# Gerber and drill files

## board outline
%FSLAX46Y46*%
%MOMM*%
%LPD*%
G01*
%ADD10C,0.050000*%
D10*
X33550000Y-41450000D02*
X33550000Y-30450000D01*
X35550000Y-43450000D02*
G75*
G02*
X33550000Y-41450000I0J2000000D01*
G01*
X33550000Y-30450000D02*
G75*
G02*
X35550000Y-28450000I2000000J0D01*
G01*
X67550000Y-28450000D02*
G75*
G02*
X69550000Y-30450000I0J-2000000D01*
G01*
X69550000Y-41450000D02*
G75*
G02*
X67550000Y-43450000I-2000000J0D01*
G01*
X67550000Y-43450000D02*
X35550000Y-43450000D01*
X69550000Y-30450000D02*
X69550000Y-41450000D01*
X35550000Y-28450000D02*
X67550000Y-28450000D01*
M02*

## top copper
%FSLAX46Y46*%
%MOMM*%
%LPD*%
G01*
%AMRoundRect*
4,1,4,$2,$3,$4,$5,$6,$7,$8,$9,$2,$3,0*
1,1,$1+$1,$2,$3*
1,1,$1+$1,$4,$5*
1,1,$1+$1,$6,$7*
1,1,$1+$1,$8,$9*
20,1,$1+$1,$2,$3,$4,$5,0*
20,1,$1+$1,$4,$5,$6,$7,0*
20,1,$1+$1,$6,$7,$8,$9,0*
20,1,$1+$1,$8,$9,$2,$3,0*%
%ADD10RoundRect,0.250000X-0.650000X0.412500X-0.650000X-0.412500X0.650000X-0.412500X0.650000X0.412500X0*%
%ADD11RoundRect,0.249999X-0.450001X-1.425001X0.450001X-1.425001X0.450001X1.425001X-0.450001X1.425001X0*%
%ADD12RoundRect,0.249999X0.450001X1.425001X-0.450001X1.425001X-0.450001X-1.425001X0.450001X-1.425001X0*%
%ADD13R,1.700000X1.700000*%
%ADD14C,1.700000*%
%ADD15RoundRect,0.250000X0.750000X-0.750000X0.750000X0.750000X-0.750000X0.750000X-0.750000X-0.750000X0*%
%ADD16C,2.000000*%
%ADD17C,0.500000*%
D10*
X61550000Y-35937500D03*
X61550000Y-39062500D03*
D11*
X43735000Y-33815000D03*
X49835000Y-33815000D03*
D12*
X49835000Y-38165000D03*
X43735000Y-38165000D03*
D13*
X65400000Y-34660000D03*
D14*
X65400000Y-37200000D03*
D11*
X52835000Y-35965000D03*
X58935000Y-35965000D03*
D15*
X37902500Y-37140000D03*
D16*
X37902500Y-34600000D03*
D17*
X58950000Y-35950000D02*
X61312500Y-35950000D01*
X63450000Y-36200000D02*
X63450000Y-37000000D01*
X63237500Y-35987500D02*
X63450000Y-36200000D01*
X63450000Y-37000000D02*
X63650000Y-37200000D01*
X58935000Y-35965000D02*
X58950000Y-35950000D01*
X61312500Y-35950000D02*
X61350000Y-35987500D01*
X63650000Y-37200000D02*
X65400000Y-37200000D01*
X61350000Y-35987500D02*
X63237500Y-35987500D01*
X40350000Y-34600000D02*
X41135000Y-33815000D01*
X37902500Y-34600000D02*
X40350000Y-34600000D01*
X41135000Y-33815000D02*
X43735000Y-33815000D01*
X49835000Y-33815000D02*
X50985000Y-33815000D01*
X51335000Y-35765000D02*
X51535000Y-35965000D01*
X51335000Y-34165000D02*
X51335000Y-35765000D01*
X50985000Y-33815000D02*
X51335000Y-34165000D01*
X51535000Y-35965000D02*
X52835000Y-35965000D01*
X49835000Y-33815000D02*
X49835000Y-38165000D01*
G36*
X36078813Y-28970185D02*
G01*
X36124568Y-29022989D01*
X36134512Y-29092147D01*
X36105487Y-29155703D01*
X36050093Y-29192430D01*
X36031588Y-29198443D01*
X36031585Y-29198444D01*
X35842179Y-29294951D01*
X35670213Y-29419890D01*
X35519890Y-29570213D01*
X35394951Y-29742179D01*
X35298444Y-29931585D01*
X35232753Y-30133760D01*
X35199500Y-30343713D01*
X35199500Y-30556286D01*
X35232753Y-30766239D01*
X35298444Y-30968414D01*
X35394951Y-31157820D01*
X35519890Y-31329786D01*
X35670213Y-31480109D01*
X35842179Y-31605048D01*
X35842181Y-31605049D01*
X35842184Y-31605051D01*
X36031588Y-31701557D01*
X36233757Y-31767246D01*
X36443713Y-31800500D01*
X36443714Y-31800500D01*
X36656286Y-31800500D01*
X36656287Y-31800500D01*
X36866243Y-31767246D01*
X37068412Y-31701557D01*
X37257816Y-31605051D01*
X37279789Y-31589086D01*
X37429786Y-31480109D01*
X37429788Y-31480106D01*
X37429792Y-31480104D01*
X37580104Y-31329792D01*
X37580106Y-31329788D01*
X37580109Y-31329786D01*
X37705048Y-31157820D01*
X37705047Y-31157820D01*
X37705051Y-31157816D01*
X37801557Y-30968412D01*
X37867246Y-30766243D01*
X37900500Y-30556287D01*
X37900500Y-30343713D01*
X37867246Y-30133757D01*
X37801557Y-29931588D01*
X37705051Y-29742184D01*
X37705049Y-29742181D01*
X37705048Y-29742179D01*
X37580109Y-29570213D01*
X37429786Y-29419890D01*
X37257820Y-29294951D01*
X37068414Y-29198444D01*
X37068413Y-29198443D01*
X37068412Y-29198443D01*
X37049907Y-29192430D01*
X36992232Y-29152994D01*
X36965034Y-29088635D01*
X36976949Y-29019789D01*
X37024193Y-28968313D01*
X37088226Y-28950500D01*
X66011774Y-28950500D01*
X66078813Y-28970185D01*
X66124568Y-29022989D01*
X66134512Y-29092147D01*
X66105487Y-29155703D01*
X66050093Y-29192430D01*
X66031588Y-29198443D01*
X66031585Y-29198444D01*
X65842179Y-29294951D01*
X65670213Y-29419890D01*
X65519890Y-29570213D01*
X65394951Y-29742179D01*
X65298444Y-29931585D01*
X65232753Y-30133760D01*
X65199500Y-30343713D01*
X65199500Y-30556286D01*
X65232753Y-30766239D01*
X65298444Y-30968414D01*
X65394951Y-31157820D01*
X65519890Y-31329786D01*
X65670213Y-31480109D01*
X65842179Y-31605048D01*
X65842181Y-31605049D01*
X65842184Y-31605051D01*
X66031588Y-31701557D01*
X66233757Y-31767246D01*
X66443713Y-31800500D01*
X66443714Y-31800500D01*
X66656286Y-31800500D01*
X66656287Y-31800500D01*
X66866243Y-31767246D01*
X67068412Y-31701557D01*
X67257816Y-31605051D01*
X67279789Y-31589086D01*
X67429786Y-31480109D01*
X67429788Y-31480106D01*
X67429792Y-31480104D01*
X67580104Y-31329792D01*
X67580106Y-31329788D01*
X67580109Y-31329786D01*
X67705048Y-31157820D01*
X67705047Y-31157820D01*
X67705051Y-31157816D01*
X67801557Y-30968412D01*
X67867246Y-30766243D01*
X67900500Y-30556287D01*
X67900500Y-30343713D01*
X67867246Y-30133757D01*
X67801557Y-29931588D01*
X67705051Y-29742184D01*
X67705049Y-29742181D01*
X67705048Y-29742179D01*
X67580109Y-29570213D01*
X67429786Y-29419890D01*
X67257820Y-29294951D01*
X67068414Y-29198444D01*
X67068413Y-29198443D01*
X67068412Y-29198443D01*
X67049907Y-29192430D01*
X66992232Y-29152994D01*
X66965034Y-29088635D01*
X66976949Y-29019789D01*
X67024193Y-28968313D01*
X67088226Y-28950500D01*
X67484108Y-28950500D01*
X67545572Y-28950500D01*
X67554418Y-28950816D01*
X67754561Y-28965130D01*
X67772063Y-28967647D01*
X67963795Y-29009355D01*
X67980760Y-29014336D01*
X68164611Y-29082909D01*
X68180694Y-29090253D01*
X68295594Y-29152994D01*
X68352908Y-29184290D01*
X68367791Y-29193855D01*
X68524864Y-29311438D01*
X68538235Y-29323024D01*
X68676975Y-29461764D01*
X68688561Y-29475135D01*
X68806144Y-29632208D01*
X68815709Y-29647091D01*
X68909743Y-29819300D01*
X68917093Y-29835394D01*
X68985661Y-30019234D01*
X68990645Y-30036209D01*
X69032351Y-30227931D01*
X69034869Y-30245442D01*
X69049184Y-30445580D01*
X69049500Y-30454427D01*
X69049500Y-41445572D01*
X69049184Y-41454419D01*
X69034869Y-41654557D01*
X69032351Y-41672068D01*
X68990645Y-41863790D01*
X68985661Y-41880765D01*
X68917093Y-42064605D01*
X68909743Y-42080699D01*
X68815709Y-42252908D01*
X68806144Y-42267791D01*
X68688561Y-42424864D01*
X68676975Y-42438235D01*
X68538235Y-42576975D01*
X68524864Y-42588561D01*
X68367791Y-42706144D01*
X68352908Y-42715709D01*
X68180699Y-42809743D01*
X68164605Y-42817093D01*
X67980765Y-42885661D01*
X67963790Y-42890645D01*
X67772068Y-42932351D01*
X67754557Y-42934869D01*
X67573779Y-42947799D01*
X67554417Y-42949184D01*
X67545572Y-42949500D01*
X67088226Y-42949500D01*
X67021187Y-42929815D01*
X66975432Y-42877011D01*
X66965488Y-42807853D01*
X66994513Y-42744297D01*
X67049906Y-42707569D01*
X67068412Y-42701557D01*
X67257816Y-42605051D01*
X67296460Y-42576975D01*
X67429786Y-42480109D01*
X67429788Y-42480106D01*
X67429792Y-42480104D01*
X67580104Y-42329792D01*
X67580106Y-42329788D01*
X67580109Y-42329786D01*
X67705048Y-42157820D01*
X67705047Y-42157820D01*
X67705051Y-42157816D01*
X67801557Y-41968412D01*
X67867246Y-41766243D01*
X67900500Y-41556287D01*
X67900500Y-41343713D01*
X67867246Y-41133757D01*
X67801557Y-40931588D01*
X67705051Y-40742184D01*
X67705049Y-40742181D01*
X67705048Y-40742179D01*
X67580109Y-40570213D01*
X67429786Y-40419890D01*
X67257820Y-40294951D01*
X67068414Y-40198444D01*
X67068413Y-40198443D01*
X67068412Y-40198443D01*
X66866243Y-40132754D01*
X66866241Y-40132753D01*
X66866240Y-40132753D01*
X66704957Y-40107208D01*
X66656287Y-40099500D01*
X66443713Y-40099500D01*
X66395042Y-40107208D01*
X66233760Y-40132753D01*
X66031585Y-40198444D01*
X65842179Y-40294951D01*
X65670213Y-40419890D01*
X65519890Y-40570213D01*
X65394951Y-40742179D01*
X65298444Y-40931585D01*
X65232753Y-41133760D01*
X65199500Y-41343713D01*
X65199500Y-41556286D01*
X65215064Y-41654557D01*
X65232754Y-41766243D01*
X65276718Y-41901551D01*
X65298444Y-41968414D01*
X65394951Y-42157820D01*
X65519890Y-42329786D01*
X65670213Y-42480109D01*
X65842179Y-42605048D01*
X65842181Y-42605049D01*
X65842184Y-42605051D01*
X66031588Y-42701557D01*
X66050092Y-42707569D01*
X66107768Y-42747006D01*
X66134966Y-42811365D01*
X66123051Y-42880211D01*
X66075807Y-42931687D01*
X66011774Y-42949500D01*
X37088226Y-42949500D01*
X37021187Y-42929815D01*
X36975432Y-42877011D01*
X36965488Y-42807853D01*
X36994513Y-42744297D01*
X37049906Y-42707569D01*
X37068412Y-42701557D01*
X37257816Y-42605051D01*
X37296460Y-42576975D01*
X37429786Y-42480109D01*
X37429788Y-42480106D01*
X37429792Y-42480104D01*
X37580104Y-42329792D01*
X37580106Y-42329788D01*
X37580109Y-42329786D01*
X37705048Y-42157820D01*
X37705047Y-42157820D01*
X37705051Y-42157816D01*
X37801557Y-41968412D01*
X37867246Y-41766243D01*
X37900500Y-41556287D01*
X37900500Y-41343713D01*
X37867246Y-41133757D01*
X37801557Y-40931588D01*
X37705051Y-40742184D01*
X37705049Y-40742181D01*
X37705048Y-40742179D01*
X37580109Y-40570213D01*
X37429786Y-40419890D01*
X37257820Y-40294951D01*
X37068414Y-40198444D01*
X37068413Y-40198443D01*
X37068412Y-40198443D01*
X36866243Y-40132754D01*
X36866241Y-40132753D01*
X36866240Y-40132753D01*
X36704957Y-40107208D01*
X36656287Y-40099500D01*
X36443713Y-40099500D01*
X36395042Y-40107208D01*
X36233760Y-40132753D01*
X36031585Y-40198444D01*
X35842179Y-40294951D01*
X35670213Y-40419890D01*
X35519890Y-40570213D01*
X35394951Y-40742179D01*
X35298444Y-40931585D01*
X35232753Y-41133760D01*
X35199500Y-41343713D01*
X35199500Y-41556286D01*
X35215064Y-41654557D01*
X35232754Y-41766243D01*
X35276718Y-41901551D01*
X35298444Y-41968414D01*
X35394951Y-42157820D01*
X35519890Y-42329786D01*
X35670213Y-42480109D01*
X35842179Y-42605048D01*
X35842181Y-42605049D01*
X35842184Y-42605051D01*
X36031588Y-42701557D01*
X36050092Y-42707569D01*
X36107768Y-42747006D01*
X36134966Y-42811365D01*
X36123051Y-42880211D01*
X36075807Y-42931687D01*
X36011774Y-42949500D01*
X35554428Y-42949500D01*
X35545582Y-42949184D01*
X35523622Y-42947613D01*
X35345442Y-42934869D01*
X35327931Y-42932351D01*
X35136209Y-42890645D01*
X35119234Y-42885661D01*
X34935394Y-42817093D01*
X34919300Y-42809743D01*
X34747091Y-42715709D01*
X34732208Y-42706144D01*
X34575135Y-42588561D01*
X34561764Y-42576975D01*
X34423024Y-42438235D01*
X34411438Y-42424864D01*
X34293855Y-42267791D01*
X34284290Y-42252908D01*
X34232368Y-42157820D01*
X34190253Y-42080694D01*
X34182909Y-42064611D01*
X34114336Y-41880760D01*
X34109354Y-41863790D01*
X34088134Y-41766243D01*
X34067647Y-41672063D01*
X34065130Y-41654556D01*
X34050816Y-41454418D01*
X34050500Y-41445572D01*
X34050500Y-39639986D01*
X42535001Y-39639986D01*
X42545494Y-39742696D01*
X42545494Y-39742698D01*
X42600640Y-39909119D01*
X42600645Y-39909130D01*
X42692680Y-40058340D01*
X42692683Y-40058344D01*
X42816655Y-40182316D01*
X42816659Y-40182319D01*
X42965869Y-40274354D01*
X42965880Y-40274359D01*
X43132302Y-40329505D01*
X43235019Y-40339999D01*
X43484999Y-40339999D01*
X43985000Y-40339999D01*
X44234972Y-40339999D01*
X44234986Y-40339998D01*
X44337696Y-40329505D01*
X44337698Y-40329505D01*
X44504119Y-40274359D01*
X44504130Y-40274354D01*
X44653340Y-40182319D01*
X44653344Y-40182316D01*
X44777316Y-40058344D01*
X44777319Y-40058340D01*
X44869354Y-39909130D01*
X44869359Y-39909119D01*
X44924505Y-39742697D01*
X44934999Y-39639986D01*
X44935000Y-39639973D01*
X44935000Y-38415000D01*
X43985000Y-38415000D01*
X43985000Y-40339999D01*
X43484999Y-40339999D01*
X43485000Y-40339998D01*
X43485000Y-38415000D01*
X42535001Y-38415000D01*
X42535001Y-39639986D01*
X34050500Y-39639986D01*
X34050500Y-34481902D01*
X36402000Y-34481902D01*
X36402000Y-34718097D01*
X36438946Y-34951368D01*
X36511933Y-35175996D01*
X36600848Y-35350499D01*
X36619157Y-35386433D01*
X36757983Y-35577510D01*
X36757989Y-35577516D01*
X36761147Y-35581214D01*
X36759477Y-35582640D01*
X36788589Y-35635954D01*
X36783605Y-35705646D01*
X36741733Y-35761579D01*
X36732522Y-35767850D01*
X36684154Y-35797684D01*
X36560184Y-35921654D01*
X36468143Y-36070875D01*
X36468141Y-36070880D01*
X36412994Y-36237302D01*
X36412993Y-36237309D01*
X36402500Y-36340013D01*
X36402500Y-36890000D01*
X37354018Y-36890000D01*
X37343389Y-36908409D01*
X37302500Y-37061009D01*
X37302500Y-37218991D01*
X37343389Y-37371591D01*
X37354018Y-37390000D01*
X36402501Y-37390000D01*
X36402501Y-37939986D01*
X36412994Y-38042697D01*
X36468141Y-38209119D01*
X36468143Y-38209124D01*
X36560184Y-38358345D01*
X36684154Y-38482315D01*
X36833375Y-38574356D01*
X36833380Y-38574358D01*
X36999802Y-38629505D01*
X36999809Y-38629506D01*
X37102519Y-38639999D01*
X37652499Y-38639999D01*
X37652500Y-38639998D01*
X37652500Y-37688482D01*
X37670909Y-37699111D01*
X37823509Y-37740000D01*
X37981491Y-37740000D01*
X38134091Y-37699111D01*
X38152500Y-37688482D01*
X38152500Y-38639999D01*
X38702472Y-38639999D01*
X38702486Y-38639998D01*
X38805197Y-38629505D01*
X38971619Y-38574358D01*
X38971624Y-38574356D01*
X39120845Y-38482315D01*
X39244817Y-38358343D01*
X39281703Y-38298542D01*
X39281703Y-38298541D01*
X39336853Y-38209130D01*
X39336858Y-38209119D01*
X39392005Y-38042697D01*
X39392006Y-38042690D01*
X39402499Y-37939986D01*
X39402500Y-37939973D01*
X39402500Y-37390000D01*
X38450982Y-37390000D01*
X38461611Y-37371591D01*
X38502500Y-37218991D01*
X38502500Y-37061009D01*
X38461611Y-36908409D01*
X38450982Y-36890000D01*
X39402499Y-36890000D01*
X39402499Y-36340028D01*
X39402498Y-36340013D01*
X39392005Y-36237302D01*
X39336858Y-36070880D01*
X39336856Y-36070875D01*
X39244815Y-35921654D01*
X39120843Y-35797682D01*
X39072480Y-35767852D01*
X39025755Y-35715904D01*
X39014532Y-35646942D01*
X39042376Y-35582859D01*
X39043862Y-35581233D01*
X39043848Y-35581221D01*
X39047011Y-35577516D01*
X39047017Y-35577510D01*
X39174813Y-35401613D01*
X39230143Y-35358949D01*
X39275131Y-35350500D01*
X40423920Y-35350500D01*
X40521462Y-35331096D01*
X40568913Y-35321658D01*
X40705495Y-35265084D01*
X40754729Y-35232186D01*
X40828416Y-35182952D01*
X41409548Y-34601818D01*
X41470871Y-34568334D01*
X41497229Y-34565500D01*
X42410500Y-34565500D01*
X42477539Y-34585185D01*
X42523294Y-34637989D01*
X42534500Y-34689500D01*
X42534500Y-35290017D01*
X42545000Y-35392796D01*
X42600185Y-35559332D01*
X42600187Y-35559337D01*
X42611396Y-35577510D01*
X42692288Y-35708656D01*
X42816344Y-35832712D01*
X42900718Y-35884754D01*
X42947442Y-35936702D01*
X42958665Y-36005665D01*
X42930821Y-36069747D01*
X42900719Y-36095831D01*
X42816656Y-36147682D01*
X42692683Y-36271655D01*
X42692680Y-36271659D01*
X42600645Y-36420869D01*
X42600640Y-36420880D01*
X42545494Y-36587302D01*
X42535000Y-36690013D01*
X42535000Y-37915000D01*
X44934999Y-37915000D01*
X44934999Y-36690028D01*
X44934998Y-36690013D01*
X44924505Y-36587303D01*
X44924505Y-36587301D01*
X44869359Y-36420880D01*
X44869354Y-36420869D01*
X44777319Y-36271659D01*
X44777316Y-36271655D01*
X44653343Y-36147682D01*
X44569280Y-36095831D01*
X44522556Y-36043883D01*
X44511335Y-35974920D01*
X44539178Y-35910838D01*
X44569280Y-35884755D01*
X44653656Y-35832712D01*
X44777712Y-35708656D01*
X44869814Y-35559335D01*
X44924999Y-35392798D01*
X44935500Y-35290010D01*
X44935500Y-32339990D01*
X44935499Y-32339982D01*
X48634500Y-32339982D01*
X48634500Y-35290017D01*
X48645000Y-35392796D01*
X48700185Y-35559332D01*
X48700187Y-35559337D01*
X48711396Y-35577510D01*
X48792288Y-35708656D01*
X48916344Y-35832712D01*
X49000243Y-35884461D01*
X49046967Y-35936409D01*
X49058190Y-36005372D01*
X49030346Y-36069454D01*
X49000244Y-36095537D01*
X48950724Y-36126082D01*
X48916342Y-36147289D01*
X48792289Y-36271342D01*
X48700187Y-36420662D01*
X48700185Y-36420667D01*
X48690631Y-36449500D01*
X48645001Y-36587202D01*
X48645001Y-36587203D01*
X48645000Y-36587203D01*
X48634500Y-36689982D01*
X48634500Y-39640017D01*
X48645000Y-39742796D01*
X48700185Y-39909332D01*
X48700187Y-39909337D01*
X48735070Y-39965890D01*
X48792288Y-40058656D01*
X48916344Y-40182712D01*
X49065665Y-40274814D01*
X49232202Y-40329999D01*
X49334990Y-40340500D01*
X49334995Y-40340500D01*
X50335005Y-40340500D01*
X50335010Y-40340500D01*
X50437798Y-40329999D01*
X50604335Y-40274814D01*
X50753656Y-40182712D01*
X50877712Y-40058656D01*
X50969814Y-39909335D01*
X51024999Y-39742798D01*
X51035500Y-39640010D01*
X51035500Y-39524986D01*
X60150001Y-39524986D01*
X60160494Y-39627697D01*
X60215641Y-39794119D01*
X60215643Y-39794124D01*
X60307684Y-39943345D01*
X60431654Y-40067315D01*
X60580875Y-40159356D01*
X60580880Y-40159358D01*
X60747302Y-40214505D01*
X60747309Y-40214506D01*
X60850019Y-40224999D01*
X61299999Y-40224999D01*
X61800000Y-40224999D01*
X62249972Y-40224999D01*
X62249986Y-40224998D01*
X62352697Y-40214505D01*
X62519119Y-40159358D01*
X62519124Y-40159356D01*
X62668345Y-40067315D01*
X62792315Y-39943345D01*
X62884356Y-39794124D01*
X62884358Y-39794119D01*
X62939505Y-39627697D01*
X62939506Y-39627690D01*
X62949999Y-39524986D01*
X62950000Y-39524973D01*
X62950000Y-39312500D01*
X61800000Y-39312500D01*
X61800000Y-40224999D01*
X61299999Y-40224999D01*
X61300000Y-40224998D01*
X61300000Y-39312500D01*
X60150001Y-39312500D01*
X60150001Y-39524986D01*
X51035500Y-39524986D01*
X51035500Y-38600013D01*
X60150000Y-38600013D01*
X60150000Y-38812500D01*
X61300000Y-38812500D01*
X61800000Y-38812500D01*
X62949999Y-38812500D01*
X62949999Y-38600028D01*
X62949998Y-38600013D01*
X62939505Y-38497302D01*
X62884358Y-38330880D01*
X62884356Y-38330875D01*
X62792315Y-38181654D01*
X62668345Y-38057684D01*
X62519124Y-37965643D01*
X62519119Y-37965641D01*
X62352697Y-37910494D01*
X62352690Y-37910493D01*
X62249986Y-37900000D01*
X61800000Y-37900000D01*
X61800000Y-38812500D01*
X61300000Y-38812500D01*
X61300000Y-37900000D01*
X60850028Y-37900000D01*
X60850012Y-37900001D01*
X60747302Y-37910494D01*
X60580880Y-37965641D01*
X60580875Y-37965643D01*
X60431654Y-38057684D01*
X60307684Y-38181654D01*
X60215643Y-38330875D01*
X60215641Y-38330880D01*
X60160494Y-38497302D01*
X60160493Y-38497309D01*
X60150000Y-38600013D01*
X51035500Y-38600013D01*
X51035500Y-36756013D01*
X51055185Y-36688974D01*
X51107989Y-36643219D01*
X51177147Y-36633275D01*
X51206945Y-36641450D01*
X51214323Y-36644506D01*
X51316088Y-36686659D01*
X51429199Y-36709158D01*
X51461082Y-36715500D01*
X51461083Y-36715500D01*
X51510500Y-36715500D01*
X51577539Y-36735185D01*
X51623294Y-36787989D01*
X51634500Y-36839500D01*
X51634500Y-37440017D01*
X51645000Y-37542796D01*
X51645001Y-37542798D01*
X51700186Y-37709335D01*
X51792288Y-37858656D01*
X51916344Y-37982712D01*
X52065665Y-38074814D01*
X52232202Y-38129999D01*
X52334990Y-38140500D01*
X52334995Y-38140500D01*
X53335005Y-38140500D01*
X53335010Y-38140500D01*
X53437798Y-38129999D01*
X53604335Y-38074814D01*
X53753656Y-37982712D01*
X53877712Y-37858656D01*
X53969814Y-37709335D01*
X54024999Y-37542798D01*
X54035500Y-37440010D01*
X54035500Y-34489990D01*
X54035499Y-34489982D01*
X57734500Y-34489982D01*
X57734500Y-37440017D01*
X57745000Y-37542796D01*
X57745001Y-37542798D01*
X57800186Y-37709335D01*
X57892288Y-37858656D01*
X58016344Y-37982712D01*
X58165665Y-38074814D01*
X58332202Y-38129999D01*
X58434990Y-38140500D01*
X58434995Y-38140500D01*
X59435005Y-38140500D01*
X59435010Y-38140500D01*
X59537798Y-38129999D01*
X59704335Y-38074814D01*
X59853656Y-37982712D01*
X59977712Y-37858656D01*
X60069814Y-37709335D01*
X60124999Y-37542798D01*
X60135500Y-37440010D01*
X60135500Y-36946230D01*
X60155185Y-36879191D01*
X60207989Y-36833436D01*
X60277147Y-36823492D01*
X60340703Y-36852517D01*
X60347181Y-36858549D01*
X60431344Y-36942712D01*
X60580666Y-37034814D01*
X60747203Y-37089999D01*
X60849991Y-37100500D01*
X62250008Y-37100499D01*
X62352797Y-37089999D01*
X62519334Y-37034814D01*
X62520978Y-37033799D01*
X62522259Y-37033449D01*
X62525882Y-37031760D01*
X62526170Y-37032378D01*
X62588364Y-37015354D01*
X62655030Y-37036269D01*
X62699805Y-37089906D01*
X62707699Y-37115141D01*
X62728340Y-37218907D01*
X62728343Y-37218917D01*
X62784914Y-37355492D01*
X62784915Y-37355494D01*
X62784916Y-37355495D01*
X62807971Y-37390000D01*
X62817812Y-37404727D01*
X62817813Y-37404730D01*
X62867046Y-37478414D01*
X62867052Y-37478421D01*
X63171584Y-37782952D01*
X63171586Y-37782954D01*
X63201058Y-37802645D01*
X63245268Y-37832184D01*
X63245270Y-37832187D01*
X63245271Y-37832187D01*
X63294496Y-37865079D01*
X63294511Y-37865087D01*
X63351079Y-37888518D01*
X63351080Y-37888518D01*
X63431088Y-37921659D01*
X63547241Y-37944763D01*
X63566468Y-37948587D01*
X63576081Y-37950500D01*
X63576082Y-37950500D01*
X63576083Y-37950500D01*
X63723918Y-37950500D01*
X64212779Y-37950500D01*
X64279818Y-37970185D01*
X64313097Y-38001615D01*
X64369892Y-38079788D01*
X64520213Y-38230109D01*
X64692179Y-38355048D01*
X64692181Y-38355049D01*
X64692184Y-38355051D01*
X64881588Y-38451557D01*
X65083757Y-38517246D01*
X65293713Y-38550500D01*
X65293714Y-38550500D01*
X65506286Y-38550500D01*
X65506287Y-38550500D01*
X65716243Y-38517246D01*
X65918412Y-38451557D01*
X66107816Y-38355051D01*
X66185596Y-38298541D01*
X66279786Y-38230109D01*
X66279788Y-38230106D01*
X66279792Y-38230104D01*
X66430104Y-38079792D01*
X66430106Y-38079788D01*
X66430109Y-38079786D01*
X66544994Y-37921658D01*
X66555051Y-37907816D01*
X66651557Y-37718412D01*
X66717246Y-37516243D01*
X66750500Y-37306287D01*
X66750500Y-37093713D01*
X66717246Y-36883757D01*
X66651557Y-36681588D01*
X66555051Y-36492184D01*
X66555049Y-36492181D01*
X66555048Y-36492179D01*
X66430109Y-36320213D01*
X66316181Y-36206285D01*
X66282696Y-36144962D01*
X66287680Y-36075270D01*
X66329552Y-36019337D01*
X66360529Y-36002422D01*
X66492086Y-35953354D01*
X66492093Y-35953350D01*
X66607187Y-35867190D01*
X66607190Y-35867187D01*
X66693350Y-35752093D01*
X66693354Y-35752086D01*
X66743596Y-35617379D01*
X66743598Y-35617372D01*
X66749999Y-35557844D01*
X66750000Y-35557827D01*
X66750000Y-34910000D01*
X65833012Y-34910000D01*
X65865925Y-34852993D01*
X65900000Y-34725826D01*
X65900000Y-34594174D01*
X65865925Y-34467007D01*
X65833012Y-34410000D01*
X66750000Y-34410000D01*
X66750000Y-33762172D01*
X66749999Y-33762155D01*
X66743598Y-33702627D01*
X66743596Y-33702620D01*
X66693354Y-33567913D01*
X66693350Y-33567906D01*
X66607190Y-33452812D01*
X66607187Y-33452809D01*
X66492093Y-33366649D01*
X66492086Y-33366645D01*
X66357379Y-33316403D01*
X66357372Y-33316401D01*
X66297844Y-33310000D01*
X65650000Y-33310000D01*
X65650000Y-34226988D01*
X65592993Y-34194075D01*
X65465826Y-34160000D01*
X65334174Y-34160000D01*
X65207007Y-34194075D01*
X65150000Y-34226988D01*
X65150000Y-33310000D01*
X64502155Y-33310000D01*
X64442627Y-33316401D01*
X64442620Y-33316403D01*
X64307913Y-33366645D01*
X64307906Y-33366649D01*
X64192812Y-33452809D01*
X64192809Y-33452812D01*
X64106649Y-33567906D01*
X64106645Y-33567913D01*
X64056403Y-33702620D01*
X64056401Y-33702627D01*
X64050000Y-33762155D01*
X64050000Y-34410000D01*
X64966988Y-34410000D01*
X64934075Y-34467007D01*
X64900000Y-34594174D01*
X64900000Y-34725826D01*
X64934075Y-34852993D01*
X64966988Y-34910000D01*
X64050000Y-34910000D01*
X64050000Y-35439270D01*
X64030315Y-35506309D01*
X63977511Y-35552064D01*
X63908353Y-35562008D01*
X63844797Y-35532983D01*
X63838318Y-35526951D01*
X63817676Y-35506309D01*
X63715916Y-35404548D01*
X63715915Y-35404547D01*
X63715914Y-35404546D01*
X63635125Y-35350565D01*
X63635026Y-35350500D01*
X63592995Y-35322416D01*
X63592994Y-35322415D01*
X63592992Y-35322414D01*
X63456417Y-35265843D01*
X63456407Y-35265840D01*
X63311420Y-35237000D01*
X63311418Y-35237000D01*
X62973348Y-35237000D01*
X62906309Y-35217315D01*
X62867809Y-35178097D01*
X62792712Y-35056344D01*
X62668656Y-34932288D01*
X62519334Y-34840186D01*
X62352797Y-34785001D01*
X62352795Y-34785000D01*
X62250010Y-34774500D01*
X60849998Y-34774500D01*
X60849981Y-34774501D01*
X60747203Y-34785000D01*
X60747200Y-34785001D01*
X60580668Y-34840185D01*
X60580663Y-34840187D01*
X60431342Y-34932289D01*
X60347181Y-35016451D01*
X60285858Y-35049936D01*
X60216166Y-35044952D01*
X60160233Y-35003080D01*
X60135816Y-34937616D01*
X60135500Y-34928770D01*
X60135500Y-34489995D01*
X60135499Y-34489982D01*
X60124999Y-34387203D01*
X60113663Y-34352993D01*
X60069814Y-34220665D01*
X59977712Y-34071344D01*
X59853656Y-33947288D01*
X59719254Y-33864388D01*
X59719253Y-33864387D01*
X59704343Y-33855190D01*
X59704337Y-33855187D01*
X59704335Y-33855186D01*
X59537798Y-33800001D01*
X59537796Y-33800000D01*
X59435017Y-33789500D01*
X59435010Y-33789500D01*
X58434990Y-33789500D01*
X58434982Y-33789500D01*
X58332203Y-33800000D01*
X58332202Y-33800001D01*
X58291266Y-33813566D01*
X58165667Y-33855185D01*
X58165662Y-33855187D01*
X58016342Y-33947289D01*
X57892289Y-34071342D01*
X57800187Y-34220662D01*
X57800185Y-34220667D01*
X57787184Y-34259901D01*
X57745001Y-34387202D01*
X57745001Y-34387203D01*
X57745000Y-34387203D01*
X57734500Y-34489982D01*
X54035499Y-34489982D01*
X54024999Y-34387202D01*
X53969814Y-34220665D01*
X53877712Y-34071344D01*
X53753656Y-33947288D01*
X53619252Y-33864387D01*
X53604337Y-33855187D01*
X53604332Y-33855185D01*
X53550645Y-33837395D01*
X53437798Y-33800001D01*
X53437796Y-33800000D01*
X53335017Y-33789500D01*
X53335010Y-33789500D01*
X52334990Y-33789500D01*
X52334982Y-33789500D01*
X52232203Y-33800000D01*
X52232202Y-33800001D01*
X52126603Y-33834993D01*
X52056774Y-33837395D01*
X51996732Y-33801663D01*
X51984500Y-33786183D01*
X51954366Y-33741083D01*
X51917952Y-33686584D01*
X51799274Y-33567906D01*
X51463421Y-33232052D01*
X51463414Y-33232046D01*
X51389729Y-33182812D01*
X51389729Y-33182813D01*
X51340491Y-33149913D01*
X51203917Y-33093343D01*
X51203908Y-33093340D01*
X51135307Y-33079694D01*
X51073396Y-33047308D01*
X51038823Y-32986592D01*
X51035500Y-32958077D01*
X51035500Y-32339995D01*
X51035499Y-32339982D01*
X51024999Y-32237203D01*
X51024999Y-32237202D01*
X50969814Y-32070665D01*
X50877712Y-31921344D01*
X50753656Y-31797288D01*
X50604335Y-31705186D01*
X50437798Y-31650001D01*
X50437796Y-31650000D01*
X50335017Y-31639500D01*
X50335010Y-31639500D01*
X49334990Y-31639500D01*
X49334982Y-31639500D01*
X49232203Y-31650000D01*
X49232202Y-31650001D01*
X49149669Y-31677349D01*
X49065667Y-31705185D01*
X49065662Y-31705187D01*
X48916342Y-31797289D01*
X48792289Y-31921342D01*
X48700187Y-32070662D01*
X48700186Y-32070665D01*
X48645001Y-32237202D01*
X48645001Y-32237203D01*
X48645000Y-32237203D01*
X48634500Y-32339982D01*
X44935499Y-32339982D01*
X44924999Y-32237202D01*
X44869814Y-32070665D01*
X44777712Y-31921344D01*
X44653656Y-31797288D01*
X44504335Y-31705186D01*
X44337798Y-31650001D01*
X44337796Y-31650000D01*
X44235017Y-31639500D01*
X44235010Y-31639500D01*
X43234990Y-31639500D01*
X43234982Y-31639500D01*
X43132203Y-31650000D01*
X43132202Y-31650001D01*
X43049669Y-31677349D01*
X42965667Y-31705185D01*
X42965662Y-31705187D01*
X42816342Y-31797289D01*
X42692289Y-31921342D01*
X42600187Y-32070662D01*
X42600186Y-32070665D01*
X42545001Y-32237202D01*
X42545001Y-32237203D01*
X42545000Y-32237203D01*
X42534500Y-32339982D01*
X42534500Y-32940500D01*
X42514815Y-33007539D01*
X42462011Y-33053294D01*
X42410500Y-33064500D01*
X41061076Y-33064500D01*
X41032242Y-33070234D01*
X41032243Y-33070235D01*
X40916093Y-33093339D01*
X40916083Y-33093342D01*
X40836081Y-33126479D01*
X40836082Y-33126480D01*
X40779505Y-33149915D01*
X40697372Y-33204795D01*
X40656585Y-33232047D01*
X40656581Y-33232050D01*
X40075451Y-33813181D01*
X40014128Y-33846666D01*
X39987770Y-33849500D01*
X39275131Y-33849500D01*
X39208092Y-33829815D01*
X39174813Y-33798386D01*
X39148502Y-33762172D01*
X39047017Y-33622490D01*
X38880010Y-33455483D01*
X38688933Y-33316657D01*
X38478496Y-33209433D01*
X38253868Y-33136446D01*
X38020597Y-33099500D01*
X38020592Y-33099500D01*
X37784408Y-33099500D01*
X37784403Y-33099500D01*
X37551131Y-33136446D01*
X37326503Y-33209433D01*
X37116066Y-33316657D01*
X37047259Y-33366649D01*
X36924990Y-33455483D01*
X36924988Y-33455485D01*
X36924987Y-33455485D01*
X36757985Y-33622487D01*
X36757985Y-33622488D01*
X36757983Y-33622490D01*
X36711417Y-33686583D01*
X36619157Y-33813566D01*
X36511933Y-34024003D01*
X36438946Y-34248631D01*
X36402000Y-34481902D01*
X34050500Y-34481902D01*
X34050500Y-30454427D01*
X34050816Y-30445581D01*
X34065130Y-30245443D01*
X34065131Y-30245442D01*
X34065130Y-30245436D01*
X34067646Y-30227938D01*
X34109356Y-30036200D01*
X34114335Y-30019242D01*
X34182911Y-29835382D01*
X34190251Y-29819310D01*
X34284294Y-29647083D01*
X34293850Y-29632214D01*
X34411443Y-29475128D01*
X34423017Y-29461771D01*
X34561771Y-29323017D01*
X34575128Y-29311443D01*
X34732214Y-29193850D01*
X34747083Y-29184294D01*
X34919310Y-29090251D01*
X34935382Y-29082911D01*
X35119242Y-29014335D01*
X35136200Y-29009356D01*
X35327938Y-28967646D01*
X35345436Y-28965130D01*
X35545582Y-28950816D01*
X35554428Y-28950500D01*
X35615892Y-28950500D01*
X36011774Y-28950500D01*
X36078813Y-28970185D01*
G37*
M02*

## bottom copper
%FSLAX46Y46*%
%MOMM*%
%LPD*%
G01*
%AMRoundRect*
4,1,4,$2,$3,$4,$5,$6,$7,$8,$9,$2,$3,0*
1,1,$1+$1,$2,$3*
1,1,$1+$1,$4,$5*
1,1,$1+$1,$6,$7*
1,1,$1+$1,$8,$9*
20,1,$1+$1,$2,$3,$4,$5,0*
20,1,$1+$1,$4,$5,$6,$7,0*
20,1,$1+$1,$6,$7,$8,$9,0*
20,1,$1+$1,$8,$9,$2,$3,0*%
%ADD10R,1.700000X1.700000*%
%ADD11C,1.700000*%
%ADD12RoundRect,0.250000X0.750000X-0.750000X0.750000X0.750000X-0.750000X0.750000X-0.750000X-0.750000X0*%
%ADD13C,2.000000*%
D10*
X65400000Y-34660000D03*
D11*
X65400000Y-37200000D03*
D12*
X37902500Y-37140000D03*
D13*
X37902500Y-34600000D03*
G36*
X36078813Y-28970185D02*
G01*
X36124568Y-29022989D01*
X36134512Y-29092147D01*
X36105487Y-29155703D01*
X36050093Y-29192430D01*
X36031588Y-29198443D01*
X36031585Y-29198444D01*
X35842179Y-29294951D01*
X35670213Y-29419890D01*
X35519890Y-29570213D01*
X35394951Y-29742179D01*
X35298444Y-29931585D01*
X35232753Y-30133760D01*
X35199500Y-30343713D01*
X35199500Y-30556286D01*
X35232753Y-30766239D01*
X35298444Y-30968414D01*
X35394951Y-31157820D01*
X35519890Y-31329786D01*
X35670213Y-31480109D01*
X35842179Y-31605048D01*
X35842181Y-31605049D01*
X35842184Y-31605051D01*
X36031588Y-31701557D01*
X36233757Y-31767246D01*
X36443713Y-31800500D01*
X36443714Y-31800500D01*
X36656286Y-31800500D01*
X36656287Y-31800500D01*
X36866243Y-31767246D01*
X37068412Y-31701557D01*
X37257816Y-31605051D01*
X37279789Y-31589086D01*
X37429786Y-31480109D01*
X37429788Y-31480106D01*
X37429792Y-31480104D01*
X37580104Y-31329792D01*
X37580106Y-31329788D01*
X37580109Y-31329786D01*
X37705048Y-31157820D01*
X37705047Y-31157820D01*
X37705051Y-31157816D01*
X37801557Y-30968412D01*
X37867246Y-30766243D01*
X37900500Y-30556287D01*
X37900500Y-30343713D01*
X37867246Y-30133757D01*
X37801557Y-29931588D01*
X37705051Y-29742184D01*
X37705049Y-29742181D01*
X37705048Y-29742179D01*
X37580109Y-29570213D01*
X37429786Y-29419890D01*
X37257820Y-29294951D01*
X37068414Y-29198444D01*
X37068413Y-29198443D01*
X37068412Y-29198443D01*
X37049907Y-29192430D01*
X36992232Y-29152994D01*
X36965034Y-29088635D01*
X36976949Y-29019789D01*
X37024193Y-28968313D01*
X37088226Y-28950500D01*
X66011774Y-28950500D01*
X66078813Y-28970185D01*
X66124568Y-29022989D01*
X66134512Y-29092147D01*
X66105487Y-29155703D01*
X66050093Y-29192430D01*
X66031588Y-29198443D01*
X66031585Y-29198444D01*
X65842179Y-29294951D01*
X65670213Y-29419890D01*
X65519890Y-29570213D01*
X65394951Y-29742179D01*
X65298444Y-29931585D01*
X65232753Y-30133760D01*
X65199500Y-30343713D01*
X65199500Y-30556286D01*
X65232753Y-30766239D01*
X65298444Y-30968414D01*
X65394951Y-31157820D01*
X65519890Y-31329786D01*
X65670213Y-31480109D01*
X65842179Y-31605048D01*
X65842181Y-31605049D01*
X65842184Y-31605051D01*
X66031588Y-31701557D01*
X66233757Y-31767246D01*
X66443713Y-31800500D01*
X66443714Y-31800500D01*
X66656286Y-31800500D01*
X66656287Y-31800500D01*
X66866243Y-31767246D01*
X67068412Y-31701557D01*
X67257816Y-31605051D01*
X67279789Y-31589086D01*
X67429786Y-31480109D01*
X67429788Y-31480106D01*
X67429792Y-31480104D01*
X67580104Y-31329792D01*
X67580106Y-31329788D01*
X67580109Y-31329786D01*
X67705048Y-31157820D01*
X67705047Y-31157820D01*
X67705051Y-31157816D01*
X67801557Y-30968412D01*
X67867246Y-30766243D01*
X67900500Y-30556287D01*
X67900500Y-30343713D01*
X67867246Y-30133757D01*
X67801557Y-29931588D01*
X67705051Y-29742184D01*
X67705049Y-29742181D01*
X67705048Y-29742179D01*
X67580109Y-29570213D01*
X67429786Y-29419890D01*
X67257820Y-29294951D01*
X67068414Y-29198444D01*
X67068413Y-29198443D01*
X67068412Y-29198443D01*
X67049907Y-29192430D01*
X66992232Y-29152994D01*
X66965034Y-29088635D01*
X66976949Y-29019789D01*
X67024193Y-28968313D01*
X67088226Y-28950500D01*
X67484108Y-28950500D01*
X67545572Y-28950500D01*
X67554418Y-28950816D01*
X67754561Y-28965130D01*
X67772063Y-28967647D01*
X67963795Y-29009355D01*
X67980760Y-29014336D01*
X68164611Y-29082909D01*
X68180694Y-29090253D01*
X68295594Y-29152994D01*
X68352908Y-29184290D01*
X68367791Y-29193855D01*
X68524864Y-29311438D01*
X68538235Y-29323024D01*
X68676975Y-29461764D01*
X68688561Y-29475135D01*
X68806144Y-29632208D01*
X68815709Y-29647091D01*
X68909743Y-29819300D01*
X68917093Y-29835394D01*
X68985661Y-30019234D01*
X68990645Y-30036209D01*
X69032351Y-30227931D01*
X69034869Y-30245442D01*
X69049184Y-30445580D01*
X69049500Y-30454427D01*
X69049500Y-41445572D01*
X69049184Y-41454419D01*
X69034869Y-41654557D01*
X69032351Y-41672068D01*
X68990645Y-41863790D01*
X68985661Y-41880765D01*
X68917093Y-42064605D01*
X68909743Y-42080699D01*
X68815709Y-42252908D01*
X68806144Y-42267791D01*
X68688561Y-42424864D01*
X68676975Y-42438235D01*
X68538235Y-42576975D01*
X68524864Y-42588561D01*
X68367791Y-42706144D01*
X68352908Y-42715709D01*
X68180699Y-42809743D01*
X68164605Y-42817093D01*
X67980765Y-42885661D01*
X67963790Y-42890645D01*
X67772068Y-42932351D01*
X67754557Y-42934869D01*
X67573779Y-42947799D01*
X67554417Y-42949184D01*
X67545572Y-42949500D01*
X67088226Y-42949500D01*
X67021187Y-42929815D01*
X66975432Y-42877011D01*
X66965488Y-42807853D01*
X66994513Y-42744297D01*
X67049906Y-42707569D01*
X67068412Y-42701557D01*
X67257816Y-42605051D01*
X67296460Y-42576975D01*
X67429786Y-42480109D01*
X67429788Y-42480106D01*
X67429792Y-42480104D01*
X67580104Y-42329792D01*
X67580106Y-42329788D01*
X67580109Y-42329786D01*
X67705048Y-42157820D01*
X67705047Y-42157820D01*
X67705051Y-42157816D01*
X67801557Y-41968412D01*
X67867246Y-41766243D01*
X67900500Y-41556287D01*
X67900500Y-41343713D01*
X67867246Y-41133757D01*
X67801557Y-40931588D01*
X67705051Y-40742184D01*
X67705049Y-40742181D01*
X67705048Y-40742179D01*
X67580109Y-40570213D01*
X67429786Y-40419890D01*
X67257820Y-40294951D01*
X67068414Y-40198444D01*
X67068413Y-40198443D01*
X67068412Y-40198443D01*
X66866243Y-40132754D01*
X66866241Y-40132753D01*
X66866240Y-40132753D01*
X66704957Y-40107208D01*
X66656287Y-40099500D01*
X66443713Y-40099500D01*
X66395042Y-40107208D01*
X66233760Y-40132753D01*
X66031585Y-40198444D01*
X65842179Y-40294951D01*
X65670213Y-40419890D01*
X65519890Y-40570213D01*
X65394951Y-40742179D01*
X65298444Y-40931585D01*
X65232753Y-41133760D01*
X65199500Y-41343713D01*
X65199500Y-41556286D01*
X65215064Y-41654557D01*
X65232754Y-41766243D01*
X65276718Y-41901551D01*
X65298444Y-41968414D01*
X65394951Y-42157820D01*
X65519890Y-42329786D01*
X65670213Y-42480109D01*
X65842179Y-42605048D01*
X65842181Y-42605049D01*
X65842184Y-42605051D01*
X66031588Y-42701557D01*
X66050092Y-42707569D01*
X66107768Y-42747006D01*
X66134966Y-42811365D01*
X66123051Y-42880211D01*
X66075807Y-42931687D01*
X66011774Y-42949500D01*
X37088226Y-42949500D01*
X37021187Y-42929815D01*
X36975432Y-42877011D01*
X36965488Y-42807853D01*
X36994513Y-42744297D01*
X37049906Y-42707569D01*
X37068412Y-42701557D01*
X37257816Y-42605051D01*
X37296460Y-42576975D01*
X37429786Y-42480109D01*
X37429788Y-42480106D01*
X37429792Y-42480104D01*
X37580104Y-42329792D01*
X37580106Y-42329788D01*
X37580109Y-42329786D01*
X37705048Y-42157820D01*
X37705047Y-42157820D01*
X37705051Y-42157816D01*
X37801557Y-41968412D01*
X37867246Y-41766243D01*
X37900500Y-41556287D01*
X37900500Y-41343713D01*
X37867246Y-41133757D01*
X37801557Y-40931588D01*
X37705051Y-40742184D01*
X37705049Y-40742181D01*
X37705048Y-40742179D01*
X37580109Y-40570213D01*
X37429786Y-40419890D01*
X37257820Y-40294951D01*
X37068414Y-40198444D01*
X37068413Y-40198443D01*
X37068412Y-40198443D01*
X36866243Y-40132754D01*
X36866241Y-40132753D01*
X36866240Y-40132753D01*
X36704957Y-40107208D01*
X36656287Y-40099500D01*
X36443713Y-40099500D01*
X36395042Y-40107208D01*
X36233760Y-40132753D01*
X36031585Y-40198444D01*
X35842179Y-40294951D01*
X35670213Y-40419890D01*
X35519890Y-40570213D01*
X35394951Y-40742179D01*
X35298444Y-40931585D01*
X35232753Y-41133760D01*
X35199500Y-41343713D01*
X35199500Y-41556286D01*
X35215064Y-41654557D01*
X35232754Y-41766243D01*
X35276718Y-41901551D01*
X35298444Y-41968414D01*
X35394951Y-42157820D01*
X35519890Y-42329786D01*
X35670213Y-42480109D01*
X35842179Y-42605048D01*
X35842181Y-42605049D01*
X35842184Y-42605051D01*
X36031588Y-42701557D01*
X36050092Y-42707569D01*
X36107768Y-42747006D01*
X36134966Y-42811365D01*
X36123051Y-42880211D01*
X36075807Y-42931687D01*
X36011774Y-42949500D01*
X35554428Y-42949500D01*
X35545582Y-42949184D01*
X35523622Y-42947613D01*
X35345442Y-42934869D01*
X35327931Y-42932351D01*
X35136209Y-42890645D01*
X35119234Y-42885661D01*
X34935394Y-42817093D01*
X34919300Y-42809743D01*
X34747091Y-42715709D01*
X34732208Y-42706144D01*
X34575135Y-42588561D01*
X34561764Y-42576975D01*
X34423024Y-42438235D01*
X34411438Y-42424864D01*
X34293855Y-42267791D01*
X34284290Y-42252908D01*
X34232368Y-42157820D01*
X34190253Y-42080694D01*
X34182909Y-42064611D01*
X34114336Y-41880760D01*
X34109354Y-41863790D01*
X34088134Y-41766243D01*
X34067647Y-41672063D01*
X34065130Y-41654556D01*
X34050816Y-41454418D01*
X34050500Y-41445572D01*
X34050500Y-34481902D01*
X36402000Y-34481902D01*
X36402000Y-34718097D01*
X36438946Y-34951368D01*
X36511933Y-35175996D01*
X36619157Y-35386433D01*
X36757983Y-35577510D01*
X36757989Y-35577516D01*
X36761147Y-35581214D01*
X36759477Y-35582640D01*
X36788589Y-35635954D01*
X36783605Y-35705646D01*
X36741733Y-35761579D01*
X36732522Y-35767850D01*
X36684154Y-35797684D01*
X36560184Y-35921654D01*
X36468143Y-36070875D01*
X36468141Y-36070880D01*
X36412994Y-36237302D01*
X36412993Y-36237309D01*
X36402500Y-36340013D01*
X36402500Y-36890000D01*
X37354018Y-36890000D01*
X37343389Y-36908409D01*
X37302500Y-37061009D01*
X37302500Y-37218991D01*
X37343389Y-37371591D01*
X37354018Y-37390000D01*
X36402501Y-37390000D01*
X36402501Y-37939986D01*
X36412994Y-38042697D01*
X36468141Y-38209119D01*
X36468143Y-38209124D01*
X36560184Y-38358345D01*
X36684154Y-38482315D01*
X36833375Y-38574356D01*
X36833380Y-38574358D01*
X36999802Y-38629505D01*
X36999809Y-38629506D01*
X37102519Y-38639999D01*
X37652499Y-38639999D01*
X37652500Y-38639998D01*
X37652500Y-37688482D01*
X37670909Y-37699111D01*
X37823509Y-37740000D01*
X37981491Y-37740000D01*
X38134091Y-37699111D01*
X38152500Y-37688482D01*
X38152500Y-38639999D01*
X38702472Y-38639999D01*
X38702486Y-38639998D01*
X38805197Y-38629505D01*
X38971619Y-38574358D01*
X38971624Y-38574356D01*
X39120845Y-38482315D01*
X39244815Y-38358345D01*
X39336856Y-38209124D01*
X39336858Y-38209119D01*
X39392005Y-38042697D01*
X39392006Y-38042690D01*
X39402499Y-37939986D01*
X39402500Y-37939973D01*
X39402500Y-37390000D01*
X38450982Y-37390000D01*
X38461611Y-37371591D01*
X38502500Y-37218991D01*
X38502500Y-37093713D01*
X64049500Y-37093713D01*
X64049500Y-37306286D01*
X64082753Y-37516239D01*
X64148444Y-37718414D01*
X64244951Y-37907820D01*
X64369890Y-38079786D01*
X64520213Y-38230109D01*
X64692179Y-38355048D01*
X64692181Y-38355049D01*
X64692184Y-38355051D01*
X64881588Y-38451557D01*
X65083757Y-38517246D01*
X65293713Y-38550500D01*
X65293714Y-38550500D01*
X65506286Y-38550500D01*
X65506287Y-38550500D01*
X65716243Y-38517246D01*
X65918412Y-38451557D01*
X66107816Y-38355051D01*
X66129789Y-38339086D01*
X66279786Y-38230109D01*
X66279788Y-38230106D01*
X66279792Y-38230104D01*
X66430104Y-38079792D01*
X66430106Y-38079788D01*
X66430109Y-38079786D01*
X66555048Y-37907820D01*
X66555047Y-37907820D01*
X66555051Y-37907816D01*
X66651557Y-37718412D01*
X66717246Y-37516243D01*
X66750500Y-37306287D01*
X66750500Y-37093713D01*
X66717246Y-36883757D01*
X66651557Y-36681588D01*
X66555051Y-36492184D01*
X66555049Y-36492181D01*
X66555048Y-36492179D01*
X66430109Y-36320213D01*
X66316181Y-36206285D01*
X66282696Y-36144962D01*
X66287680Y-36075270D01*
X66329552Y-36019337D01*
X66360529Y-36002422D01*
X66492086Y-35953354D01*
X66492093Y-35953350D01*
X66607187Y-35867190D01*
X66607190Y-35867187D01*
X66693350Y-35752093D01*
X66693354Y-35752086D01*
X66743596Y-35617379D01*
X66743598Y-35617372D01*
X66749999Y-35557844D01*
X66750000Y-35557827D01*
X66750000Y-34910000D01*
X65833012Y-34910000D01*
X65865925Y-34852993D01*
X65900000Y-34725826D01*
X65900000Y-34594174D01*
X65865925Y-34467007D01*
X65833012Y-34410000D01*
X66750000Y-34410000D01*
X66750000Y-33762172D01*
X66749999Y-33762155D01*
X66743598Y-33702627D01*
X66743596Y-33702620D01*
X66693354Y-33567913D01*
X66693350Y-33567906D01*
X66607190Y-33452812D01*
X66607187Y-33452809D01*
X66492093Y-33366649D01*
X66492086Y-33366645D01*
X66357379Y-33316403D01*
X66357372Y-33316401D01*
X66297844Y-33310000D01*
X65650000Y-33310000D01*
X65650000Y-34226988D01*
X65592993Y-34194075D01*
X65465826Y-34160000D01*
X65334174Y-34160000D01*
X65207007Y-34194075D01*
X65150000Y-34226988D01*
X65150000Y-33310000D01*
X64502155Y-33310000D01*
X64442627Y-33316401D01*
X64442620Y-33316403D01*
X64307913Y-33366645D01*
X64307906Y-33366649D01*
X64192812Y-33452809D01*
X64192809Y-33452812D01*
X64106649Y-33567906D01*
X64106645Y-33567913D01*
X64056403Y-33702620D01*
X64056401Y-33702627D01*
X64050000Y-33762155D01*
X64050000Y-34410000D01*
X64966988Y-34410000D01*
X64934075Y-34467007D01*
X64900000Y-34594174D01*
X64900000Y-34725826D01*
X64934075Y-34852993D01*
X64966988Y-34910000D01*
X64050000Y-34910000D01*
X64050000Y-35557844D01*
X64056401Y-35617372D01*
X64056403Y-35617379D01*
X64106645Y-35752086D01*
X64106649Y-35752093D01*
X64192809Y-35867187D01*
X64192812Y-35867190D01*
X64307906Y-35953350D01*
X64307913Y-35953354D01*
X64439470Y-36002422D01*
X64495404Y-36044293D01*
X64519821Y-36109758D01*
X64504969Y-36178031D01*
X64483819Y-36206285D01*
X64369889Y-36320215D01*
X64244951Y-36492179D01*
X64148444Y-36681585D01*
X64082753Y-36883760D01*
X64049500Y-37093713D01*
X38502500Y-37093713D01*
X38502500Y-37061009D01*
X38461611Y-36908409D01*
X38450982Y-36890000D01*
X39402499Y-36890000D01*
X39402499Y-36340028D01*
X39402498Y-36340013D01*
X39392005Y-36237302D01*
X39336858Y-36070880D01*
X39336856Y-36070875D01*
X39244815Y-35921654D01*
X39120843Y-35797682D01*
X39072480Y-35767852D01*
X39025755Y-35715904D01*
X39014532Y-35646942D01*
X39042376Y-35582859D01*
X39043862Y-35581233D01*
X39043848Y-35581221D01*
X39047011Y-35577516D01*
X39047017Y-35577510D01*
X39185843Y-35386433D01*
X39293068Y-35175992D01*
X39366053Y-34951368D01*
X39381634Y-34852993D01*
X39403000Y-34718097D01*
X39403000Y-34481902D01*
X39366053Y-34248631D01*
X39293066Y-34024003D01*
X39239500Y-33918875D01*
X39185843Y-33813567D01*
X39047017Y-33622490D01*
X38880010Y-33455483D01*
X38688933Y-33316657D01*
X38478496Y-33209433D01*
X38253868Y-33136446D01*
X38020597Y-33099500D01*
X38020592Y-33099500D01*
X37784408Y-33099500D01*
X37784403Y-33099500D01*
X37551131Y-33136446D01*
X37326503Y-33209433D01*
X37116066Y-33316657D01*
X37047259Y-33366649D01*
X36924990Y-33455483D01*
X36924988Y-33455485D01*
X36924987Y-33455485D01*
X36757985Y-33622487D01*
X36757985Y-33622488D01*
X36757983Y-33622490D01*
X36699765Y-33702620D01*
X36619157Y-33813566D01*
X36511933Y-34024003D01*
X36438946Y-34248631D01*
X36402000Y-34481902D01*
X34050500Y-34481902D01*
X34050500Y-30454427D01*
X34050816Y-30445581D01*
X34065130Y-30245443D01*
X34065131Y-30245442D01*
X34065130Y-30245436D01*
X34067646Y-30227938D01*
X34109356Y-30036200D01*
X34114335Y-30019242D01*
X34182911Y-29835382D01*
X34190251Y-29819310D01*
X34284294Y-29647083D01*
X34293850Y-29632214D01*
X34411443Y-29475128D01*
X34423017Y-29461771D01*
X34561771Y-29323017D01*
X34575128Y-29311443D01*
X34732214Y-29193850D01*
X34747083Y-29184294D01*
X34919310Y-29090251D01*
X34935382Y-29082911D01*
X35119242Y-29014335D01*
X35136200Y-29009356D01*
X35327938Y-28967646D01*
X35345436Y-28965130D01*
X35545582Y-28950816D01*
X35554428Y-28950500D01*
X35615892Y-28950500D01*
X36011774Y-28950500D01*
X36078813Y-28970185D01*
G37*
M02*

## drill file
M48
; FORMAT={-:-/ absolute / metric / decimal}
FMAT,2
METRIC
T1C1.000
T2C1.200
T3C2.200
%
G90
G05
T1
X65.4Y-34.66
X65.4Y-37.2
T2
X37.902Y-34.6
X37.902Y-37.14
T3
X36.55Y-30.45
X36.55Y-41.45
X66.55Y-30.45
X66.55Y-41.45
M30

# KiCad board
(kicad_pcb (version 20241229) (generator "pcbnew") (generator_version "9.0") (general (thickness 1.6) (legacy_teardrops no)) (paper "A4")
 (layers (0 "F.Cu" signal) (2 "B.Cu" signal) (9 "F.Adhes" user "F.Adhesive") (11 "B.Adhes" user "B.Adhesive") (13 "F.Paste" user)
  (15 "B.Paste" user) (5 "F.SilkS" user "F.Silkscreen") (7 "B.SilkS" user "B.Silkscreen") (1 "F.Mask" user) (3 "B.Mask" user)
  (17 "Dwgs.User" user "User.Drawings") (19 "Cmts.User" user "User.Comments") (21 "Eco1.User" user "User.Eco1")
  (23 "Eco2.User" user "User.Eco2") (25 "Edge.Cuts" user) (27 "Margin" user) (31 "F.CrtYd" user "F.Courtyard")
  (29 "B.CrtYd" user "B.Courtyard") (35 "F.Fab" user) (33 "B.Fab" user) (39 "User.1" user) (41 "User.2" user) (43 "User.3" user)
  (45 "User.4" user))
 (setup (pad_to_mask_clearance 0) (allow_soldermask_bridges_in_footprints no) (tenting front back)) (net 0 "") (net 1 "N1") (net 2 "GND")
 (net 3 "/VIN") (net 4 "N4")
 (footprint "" (layer "F.Cu") (at 36.55 30.45)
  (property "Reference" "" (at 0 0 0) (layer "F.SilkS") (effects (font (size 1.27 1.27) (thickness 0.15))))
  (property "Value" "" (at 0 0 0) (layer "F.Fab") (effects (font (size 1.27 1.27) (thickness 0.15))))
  (pad "" np_thru_hole circle (at 0 0) (size 2.2 2.2) (drill 2.2) (layers "*.Cu" "*.Mask")))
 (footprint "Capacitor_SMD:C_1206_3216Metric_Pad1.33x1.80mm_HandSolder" (layer "F.Cu") (at 61.55 37.5 -90)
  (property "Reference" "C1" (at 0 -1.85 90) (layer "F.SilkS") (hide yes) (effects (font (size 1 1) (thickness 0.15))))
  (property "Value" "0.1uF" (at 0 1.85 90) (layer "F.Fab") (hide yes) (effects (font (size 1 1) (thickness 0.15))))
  (pad "1" smd roundrect (at -1.5625 0 270) (size 1.325 1.8) (layers "F.Cu" "F.Mask" "F.Paste") (roundrect_rratio 0.188679) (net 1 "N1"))
  (pad "2" smd roundrect (at 1.5625 0 270) (size 1.325 1.8) (layers "F.Cu" "F.Mask" "F.Paste") (roundrect_rratio 0.188679) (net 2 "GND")))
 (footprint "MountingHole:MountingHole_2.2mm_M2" (layer "F.Cu") (at 66.55 41.45)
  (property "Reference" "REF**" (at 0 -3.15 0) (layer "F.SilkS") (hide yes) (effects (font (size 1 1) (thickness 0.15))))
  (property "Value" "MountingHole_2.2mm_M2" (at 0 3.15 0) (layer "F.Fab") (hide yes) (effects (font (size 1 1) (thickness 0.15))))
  (pad "" np_thru_hole circle (at 0 0) (size 2.2 2.2) (drill 2.2) (layers "*.Cu" "*.Mask")))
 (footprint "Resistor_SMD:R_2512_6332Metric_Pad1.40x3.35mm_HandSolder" (layer "F.Cu") (at 46.785 33.815)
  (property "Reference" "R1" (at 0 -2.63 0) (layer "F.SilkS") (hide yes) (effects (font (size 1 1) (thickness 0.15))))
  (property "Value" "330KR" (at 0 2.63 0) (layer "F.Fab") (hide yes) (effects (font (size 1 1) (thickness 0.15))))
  (pad "1" smd roundrect (at -3.05 0) (size 1.4 3.35) (layers "F.Cu" "F.Mask" "F.Paste") (roundrect_rratio 0.178571) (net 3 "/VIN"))
  (pad "2" smd roundrect (at 3.05 0) (size 1.4 3.35) (layers "F.Cu" "F.Mask" "F.Paste") (roundrect_rratio 0.178571) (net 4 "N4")))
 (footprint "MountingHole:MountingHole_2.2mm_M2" (layer "F.Cu") (at 66.55 30.45)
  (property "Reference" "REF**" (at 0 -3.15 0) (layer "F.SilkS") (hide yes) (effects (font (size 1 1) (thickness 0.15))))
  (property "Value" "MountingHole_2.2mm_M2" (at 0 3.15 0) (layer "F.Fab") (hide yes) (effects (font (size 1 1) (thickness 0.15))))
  (pad "" np_thru_hole circle (at 0 0) (size 2.2 2.2) (drill 2.2) (layers "*.Cu" "*.Mask")))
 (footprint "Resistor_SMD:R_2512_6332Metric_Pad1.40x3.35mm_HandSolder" (layer "F.Cu") (at 46.785 38.165 180)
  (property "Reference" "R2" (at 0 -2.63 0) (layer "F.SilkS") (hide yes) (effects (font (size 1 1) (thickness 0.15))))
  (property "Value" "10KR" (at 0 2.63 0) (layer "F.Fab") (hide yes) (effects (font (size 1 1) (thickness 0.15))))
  (pad "1" smd roundrect (at -3.05 0 180) (size 1.4 3.35) (layers "F.Cu" "F.Mask" "F.Paste") (roundrect_rratio 0.178571) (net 4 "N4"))
  (pad "2" smd roundrect (at 3.05 0 180) (size 1.4 3.35) (layers "F.Cu" "F.Mask" "F.Paste") (roundrect_rratio 0.178571) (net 2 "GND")))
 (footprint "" (layer "F.Cu") (at 36.55 41.45)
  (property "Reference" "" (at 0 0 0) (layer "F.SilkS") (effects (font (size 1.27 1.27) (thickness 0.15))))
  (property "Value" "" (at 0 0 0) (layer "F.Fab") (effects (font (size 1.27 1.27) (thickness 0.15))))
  (pad "" np_thru_hole circle (at 0 0) (size 2.2 2.2) (drill 2.2) (layers "*.Cu" "*.Mask")))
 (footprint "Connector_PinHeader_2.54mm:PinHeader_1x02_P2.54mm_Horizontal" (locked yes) (layer "F.Cu") (at 65.4 34.66)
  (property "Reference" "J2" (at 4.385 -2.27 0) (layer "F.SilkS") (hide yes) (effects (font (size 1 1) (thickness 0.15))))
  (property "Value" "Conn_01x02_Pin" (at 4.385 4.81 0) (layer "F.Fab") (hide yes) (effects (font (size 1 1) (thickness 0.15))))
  (pad "1" thru_hole rect (at 0 0) (size 1.7 1.7) (drill 1) (layers "*.Cu" "*.Mask") (remove_unused_layers no) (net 2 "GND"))
  (pad "2" thru_hole circle (at 0 2.54) (size 1.7 1.7) (drill 1) (layers "*.Cu" "*.Mask") (remove_unused_layers no) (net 1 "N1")))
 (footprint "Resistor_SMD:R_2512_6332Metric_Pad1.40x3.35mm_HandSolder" (layer "F.Cu") (at 55.885 35.965)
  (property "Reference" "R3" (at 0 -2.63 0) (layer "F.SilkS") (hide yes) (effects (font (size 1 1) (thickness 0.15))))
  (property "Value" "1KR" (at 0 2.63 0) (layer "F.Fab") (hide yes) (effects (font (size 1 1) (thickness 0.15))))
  (pad "1" smd roundrect (at -3.05 0) (size 1.4 3.35) (layers "F.Cu" "F.Mask" "F.Paste") (roundrect_rratio 0.178571) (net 4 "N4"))
  (pad "2" smd roundrect (at 3.05 0) (size 1.4 3.35) (layers "F.Cu" "F.Mask" "F.Paste") (roundrect_rratio 0.178571) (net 1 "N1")))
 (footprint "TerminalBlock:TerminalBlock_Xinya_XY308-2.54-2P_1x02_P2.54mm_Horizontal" (layer "F.Cu") (at 37.9025 37.14 90)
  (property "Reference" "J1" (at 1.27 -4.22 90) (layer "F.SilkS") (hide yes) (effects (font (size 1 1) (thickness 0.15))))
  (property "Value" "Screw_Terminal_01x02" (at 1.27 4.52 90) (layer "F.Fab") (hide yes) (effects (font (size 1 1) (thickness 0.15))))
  (pad "1" thru_hole roundrect (at 0 0 90) (size 2 2) (drill 1.2) (layers "*.Cu" "*.Mask") (remove_unused_layers no)
   (roundrect_rratio 0.125) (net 2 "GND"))
  (pad "2" thru_hole circle (at 2.54 0 90) (size 2 2) (drill 1.2) (layers "*.Cu" "*.Mask") (remove_unused_layers no) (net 3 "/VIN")))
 (gr_line (start 33.55 41.45) (end 33.55 30.45) (stroke (width 0.05) (type default)) (layer "Edge.Cuts"))
 (gr_arc (start 35.55 43.45) (mid 34.135786 42.864214) (end 33.55 41.45) (stroke (width 0.05) (type default)) (layer "Edge.Cuts"))
 (gr_arc (start 33.55 30.45) (mid 34.135786 29.035786) (end 35.55 28.45) (stroke (width 0.05) (type default)) (layer "Edge.Cuts"))
 (gr_arc (start 67.55 28.45) (mid 68.964214 29.035786) (end 69.55 30.45) (stroke (width 0.05) (type default)) (layer "Edge.Cuts"))
 (gr_arc (start 69.55 41.45) (mid 68.964214 42.864214) (end 67.55 43.45) (stroke (width 0.05) (type default)) (layer "Edge.Cuts"))
 (gr_line (start 67.55 43.45) (end 35.55 43.45) (stroke (width 0.05) (type default)) (layer "Edge.Cuts"))
 (gr_line (start 69.55 30.45) (end 69.55 41.45) (stroke (width 0.05) (type default)) (layer "Edge.Cuts"))
 (gr_line (start 35.55 28.45) (end 67.55 28.45) (stroke (width 0.05) (type default)) (layer "Edge.Cuts"))
 (segment (start 58.95 35.95) (end 61.3125 35.95) (width 0.5) (layer "F.Cu") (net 1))
 (segment (start 63.45 36.2) (end 63.45 37) (width 0.5) (layer "F.Cu") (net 1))
 (segment (start 63.2375 35.9875) (end 63.45 36.2) (width 0.5) (layer "F.Cu") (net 1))
 (segment (start 63.45 37) (end 63.65 37.2) (width 0.5) (layer "F.Cu") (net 1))
 (segment (start 58.935 35.965) (end 58.95 35.95) (width 0.5) (layer "F.Cu") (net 1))
 (segment (start 61.3125 35.95) (end 61.35 35.9875) (width 0.5) (layer "F.Cu") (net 1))
 (segment (start 63.65 37.2) (end 65.4 37.2) (width 0.5) (layer "F.Cu") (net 1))
 (segment (start 61.35 35.9875) (end 63.2375 35.9875) (width 0.5) (layer "F.Cu") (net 1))
 (segment (start 40.35 34.6) (end 41.135 33.815) (width 0.5) (layer "F.Cu") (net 3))
 (segment (start 37.9025 34.6) (end 40.35 34.6) (width 0.5) (layer "F.Cu") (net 3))
 (segment (start 41.135 33.815) (end 43.735 33.815) (width 0.5) (layer "F.Cu") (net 3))
 (segment (start 49.835 33.815) (end 50.985 33.815) (width 0.5) (layer "F.Cu") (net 4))
 (segment (start 51.335 35.765) (end 51.535 35.965) (width 0.5) (layer "F.Cu") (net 4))
 (segment (start 51.335 34.165) (end 51.335 35.765) (width 0.5) (layer "F.Cu") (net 4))
 (segment (start 50.985 33.815) (end 51.335 34.165) (width 0.5) (layer "F.Cu") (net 4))
 (segment (start 51.535 35.965) (end 52.835 35.965) (width 0.5) (layer "F.Cu") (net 4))
 (segment (start 49.835 33.815) (end 49.835 38.165) (width 0.5) (layer "F.Cu") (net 4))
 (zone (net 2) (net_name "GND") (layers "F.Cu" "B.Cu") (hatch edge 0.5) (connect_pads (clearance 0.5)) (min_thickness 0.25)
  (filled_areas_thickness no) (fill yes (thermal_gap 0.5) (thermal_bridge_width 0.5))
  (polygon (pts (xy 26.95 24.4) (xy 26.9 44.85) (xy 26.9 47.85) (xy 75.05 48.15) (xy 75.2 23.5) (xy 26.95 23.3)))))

